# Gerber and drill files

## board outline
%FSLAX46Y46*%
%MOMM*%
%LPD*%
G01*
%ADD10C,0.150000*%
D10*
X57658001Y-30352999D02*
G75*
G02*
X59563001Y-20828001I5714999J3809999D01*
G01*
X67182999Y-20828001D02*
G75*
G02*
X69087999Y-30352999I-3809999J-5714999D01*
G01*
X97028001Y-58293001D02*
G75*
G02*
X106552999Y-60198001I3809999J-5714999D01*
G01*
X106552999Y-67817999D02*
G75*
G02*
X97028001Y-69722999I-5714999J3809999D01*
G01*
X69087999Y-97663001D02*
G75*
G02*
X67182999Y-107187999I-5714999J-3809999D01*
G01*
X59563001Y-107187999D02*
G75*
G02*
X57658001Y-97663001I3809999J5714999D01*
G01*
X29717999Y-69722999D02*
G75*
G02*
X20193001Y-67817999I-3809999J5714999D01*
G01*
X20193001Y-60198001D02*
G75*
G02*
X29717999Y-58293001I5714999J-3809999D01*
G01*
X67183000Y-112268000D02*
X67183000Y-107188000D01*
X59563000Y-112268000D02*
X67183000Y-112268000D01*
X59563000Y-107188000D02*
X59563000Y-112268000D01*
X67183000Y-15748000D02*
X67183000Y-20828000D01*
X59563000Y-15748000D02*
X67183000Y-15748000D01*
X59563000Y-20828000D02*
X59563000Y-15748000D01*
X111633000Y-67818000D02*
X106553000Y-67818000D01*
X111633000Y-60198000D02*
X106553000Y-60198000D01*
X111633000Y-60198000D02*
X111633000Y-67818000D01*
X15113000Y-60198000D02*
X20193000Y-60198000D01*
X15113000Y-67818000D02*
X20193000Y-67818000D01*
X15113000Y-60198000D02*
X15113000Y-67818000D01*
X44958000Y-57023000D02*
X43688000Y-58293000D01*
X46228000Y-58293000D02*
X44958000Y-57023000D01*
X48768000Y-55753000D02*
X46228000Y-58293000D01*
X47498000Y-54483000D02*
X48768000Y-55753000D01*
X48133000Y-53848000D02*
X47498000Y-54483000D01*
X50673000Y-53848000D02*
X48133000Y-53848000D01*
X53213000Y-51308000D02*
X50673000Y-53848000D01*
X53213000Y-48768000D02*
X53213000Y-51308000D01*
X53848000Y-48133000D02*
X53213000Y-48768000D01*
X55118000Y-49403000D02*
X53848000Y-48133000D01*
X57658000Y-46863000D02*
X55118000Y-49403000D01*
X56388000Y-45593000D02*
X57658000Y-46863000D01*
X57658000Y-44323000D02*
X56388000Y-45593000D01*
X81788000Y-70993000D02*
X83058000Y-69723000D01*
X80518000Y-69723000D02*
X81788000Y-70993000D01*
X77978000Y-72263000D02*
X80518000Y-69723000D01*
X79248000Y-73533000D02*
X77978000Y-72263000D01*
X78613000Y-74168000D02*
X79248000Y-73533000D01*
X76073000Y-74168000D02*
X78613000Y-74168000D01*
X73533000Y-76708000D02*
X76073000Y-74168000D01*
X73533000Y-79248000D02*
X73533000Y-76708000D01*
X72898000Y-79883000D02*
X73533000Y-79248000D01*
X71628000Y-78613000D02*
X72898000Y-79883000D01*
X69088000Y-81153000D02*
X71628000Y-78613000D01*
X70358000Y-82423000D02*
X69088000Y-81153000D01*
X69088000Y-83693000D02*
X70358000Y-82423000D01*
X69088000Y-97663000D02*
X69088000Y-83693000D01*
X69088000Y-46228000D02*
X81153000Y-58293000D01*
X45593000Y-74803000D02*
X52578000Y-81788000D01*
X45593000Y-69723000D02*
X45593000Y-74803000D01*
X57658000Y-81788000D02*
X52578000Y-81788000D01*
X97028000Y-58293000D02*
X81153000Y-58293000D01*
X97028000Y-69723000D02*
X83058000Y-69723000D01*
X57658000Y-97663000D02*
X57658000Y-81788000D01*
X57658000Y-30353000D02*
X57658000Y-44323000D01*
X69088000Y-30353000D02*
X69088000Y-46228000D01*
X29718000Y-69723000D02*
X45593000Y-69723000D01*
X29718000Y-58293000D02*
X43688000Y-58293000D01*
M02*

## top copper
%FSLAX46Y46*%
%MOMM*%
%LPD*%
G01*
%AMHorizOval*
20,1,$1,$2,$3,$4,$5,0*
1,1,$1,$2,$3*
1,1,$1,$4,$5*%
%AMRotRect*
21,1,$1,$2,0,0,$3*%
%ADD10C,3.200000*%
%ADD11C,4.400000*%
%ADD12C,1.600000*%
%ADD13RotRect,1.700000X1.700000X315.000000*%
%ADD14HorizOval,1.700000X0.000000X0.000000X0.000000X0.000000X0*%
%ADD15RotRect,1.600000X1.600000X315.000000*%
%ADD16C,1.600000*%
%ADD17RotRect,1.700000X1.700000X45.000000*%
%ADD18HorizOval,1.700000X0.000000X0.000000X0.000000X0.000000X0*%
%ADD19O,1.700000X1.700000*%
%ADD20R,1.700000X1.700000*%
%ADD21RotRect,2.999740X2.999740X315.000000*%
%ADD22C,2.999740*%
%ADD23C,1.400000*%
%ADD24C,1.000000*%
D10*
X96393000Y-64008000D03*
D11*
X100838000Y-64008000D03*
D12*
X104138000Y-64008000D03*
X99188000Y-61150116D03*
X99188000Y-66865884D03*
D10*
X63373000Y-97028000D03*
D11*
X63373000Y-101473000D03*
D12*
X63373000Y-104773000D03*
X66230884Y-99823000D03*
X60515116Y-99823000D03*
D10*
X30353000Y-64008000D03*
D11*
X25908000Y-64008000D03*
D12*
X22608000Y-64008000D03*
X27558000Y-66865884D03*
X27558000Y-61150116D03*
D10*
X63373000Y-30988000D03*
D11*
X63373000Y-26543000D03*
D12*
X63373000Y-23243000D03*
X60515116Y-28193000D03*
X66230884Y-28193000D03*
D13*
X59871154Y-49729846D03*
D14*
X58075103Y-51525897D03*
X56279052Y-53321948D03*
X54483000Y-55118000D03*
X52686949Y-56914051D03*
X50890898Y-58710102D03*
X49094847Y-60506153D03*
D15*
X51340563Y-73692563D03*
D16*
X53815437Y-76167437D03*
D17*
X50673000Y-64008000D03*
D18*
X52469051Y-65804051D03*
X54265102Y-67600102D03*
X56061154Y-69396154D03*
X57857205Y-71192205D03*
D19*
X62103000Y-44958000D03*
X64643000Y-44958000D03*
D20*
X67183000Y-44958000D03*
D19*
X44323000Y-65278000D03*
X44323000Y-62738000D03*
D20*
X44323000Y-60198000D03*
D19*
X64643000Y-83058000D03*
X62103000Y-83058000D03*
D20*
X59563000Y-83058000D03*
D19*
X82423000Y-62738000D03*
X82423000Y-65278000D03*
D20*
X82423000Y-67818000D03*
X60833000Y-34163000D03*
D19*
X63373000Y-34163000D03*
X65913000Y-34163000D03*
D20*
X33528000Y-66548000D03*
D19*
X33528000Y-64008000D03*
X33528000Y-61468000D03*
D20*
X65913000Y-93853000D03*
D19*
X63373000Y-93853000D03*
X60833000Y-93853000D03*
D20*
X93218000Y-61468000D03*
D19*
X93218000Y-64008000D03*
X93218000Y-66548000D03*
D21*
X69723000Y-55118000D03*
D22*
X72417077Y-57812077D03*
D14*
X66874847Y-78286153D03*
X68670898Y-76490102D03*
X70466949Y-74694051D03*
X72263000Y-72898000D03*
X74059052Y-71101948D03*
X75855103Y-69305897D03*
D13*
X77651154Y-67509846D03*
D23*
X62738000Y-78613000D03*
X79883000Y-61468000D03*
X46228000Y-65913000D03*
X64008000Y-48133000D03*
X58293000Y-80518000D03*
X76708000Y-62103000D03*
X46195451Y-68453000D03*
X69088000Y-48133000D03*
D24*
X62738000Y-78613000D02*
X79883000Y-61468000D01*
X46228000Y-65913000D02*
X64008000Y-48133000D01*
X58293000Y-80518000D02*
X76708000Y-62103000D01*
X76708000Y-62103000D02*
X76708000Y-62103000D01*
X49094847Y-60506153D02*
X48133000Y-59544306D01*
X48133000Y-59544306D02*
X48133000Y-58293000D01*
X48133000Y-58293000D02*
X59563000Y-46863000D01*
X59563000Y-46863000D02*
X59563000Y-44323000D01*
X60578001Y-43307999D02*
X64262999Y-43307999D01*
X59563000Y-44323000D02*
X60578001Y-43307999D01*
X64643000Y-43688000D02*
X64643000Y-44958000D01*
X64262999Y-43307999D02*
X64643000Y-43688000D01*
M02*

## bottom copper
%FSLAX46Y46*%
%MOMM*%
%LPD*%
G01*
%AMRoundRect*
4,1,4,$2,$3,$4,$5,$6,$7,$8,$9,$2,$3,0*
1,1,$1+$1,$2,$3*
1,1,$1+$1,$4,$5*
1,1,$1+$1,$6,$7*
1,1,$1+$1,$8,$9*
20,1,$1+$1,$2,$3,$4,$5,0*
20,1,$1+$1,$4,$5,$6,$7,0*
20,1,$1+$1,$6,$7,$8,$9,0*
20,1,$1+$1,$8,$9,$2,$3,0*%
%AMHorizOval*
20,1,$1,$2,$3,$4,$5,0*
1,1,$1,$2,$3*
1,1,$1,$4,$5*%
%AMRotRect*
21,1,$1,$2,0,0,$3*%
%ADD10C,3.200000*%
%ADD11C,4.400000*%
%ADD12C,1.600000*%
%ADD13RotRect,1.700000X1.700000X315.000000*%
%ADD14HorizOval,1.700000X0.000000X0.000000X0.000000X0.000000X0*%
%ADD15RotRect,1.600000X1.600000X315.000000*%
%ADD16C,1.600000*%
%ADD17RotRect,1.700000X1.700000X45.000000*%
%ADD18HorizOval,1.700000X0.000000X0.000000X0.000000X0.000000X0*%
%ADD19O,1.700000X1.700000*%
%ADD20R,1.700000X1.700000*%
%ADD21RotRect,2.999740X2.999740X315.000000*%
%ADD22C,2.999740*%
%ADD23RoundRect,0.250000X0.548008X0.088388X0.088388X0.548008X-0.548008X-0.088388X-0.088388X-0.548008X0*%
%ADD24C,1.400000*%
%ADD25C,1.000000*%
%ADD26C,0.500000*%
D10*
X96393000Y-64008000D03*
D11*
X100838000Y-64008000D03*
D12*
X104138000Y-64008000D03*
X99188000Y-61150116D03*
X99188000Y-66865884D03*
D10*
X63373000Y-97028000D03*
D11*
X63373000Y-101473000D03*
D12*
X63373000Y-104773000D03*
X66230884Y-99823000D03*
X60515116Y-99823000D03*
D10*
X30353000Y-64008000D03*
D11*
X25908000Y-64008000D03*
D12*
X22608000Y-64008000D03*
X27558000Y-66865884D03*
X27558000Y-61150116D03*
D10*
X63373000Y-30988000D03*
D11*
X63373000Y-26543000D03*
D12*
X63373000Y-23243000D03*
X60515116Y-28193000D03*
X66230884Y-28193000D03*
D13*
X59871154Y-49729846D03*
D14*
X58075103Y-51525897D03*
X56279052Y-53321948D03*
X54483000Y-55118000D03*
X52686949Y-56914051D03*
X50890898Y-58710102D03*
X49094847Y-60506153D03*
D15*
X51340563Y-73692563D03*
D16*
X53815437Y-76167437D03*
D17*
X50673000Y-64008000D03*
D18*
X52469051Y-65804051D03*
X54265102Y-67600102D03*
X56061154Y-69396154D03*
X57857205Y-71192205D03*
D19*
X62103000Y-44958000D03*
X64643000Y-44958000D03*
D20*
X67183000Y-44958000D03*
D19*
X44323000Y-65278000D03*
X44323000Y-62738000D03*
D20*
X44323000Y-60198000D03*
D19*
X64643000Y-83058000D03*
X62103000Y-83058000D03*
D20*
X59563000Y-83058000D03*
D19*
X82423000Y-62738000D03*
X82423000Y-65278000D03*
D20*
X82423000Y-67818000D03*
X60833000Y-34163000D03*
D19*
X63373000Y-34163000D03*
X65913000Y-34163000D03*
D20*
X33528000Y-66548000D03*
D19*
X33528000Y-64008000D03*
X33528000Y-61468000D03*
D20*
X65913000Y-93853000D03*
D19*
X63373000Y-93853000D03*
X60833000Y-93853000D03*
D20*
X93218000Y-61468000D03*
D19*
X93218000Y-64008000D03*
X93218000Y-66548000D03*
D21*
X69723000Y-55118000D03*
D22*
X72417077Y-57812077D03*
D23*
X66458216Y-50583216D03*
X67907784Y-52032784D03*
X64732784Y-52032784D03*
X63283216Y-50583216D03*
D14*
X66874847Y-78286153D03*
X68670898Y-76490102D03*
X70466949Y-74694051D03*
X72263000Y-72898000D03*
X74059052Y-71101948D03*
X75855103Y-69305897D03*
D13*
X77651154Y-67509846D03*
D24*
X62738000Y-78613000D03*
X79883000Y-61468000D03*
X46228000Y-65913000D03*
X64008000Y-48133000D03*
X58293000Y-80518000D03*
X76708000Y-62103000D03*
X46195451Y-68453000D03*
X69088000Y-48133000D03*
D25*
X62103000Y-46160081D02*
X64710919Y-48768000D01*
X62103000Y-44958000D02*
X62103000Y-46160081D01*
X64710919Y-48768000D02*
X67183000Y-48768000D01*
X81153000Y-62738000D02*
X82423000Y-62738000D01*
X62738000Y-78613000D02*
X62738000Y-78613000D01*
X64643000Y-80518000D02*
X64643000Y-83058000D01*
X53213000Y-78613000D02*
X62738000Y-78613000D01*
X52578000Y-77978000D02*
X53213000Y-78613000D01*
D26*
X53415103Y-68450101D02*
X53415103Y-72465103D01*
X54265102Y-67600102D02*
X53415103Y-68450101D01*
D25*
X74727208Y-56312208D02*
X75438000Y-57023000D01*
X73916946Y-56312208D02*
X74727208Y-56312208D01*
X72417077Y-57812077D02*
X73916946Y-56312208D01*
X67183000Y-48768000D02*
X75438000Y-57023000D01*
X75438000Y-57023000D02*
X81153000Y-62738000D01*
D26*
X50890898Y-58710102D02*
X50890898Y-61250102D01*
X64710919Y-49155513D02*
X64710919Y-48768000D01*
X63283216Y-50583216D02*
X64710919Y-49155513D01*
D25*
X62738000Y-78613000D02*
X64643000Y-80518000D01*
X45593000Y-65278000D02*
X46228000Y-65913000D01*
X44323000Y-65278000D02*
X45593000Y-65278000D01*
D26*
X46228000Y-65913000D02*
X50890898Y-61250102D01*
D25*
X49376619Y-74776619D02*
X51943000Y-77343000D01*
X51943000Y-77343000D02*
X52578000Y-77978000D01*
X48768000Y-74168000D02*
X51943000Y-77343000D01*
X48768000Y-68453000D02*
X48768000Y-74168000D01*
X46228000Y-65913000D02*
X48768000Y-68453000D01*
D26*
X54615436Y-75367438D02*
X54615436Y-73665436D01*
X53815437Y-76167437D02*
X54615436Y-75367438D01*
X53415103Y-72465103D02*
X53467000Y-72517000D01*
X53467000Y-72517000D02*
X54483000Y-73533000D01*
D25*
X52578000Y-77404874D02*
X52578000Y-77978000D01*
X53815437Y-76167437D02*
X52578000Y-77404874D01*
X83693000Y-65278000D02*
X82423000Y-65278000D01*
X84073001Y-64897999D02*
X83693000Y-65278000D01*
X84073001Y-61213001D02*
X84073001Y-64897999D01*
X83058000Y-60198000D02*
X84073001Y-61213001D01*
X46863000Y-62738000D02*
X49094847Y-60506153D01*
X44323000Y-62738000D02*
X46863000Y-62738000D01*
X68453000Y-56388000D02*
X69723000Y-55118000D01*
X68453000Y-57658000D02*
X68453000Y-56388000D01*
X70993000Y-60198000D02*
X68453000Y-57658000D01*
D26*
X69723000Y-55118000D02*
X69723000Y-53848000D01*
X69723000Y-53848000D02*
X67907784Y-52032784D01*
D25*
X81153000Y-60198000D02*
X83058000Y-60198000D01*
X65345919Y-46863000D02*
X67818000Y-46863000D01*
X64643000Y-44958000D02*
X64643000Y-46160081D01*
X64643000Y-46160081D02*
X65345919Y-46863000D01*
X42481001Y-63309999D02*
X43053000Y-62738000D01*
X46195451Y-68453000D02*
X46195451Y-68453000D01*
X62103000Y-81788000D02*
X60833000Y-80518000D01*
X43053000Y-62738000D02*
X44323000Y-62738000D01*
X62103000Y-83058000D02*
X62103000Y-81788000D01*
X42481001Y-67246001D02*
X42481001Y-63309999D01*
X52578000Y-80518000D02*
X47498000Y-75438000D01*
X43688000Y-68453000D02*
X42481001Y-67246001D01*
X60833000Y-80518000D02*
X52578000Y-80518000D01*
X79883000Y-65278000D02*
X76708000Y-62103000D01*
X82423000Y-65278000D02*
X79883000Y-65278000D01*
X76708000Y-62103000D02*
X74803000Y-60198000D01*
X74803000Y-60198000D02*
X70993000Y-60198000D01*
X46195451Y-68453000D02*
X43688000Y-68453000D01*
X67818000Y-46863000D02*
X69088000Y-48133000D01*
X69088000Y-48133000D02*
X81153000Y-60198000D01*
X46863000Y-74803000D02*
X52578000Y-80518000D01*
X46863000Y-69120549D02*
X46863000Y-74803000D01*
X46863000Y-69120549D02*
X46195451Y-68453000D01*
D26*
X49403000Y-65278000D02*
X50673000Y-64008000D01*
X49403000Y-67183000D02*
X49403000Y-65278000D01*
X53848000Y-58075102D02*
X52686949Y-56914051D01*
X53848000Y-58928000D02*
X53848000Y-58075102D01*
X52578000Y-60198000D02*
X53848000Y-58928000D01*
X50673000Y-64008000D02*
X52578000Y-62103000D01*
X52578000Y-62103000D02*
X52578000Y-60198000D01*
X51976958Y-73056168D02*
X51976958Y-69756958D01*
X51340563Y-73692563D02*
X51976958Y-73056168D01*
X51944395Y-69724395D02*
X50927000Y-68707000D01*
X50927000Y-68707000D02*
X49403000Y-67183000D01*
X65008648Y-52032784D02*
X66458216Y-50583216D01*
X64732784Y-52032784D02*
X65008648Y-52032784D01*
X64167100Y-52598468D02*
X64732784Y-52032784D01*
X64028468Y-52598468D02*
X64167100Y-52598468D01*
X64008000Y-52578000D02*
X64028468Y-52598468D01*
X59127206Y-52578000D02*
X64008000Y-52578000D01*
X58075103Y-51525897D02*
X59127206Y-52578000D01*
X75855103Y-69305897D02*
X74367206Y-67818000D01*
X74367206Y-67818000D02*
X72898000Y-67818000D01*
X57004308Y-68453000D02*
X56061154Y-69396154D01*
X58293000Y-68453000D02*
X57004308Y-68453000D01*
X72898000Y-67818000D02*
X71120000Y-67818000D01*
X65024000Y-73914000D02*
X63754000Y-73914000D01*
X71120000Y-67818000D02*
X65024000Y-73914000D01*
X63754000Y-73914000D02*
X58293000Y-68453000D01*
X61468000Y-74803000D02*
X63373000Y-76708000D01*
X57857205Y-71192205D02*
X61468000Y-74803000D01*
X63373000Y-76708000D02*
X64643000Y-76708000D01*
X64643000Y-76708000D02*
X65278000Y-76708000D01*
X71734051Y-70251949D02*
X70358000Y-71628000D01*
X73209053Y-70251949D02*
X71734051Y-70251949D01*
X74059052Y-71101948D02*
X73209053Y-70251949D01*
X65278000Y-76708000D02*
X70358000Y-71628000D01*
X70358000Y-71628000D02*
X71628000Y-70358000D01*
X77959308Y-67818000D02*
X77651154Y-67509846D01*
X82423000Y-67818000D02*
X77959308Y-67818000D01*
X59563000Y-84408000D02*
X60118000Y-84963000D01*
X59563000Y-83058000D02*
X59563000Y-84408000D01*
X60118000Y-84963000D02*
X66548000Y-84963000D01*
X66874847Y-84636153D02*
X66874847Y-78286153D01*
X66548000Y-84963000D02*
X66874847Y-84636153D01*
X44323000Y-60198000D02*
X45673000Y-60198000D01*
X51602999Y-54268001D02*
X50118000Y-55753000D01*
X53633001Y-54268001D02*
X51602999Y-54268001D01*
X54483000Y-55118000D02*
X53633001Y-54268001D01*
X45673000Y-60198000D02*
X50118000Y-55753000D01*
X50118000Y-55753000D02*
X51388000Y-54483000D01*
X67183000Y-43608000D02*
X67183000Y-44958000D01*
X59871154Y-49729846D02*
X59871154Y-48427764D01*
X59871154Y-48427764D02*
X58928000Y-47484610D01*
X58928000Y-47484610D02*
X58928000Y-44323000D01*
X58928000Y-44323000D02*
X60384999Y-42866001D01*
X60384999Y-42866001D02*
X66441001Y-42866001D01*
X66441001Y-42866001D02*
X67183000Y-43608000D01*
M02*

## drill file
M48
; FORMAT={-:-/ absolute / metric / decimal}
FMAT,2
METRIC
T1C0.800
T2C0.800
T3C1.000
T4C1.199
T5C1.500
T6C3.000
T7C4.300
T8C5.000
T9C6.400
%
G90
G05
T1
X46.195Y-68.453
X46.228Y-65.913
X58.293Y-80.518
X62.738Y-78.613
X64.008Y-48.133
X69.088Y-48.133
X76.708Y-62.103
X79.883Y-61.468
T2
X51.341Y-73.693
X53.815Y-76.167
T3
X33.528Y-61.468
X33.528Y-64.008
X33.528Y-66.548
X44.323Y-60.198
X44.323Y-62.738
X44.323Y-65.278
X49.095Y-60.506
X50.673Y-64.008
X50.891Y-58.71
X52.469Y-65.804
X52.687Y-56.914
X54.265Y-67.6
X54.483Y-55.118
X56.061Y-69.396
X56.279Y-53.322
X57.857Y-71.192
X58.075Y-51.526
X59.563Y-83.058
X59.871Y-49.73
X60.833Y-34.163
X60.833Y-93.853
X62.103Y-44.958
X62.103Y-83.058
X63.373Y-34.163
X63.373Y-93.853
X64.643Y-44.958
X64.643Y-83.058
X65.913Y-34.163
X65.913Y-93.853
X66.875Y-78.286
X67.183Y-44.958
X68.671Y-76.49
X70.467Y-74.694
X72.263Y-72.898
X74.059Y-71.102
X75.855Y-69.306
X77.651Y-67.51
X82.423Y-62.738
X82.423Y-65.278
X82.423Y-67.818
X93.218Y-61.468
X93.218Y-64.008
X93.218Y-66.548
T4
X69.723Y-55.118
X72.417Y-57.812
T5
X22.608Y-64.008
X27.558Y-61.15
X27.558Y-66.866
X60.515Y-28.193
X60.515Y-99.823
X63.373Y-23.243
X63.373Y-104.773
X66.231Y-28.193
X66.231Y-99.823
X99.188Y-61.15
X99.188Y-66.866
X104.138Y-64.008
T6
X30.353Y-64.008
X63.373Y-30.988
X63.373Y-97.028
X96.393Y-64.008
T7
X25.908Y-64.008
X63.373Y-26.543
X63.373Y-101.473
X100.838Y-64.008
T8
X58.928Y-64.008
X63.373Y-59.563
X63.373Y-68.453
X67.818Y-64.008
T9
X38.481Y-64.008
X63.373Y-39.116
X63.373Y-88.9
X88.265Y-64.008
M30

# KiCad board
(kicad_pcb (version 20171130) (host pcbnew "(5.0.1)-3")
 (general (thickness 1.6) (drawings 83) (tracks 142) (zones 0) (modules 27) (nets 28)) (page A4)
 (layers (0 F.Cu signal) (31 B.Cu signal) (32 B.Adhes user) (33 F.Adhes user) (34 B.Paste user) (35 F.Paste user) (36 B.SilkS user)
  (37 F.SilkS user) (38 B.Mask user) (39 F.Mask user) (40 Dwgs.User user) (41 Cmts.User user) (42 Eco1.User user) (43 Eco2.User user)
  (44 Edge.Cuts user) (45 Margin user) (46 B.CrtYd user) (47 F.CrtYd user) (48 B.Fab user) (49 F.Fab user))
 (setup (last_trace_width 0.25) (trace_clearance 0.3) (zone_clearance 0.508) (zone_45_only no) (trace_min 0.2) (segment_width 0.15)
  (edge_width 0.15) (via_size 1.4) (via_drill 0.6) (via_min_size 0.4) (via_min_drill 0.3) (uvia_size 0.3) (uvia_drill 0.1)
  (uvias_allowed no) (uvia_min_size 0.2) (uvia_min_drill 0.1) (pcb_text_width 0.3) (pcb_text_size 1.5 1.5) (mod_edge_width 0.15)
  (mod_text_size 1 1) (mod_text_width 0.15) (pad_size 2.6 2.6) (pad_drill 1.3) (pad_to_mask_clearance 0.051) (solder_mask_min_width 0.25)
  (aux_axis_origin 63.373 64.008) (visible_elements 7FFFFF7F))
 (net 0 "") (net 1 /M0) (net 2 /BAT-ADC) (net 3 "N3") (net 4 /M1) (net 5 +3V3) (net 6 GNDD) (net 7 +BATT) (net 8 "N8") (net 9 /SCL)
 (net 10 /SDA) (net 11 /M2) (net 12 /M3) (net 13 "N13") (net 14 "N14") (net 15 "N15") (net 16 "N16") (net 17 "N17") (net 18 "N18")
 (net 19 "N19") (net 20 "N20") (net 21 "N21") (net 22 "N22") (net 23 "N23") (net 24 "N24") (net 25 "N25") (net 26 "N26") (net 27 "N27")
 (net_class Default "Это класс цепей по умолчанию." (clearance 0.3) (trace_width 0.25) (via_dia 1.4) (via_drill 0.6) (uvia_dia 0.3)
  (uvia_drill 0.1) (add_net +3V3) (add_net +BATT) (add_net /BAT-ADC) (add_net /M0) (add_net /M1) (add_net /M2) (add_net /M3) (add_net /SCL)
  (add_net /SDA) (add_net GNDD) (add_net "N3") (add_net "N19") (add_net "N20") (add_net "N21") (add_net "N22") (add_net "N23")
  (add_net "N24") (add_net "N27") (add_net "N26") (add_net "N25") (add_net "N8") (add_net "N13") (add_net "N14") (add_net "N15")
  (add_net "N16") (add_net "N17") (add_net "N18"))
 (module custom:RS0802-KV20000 (layer F.Cu) (at 100.838 64.008)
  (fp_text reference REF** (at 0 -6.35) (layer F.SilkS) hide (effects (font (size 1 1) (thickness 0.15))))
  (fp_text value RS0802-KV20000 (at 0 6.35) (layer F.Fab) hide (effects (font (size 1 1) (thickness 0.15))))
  (pad "" np_thru_hole circle (at -4.445 0) (size 3.2 3.2) (drill 3) (layers *.Cu *.Mask))
  (pad "" np_thru_hole circle (at 0 0) (size 4.4 4.4) (drill 4.3) (layers *.Cu *.Mask))
  (pad "" np_thru_hole circle (at 3.3 0) (size 1.6 1.6) (drill 1.5) (layers *.Cu *.Mask))
  (pad "" np_thru_hole circle (at -1.65 -2.857884 120) (size 1.6 1.6) (drill 1.5) (layers *.Cu *.Mask))
  (pad "" np_thru_hole circle (at -1.65 2.857884 240) (size 1.6 1.6) (drill 1.5) (layers *.Cu *.Mask)))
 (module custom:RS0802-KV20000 (layer F.Cu) (at 63.373 101.473 270)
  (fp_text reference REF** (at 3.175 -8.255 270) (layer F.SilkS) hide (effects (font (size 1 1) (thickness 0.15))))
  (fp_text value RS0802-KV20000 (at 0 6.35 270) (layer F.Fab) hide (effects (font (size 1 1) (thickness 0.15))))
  (pad "" np_thru_hole circle (at -4.445 0 270) (size 3.2 3.2) (drill 3) (layers *.Cu *.Mask))
  (pad "" np_thru_hole circle (at 0 0 270) (size 4.4 4.4) (drill 4.3) (layers *.Cu *.Mask))
  (pad "" np_thru_hole circle (at 3.3 0 270) (size 1.6 1.6) (drill 1.5) (layers *.Cu *.Mask))
  (pad "" np_thru_hole circle (at -1.65 -2.857884 30) (size 1.6 1.6) (drill 1.5) (layers *.Cu *.Mask))
  (pad "" np_thru_hole circle (at -1.65 2.857884 150) (size 1.6 1.6) (drill 1.5) (layers *.Cu *.Mask)))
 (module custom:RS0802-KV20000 (layer F.Cu) (at 25.908 64.008 180)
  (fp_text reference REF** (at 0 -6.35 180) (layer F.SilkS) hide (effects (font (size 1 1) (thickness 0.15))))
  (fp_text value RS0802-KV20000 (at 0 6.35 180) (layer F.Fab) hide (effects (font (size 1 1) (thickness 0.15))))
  (pad "" np_thru_hole circle (at -4.445 0 180) (size 3.2 3.2) (drill 3) (layers *.Cu *.Mask))
  (pad "" np_thru_hole circle (at 0 0 180) (size 4.4 4.4) (drill 4.3) (layers *.Cu *.Mask))
  (pad "" np_thru_hole circle (at 3.3 0 180) (size 1.6 1.6) (drill 1.5) (layers *.Cu *.Mask))
  (pad "" np_thru_hole circle (at -1.65 -2.857884 300) (size 1.6 1.6) (drill 1.5) (layers *.Cu *.Mask))
  (pad "" np_thru_hole circle (at -1.65 2.857884 60) (size 1.6 1.6) (drill 1.5) (layers *.Cu *.Mask)))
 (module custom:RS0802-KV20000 (layer F.Cu) (at 63.373 26.543 90)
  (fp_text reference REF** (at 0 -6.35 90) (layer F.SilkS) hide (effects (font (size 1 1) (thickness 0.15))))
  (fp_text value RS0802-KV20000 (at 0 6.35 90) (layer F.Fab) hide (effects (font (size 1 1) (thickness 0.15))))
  (pad "" np_thru_hole circle (at -4.445 0 90) (size 3.2 3.2) (drill 3) (layers *.Cu *.Mask))
  (pad "" np_thru_hole circle (at 0 0 90) (size 4.4 4.4) (drill 4.3) (layers *.Cu *.Mask))
  (pad "" np_thru_hole circle (at 3.3 0 90) (size 1.6 1.6) (drill 1.5) (layers *.Cu *.Mask))
  (pad "" np_thru_hole circle (at -1.65 -2.857884 210) (size 1.6 1.6) (drill 1.5) (layers *.Cu *.Mask))
  (pad "" np_thru_hole circle (at -1.65 2.857884 330) (size 1.6 1.6) (drill 1.5) (layers *.Cu *.Mask)))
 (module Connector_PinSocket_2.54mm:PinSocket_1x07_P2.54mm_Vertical (layer F.Cu) (at 59.871154 49.729846 315)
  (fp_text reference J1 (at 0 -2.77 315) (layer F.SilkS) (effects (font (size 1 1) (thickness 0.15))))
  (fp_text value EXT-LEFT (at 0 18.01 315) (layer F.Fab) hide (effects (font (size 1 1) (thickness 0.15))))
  (pad 1 thru_hole rect (at 0 0 315) (size 1.7 1.7) (drill 1) (layers *.Cu *.Mask) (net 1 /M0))
  (pad 2 thru_hole oval (at 0 2.54 315) (size 1.7 1.7) (drill 1) (layers *.Cu *.Mask) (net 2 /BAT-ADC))
  (pad 3 thru_hole oval (at 0 5.079999 315) (size 1.7 1.7) (drill 1) (layers *.Cu *.Mask) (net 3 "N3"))
  (pad 4 thru_hole oval (at 0 7.62 315) (size 1.7 1.7) (drill 1) (layers *.Cu *.Mask) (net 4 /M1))
  (pad 5 thru_hole oval (at 0 10.16 315) (size 1.7 1.7) (drill 1) (layers *.Cu *.Mask) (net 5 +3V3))
  (pad 6 thru_hole oval (at 0 12.7 315) (size 1.7 1.7) (drill 1) (layers *.Cu *.Mask) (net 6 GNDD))
  (pad 7 thru_hole oval (at 0 15.24 315) (size 1.7 1.7) (drill 1) (layers *.Cu *.Mask) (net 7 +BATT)))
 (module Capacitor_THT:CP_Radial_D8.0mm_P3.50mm (layer F.Cu) (at 52.578 74.93 315)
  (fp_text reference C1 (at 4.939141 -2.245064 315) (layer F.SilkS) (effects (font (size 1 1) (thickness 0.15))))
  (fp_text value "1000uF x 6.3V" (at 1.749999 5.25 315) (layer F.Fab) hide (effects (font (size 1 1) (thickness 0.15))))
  (pad 1 thru_hole rect (at -1.75 0 315) (size 1.6 1.6) (drill 0.8) (layers *.Cu *.Mask) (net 5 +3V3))
  (pad 2 thru_hole circle (at 1.75 0 315) (size 1.6 1.6) (drill 0.8) (layers *.Cu *.Mask) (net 6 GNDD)))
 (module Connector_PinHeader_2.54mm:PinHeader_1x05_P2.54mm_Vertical (layer F.Cu) (at 50.673 64.008 45)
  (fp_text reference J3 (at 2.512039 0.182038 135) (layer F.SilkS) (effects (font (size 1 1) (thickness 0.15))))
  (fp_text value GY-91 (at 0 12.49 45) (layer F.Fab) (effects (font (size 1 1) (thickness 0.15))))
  (pad 1 thru_hole rect (at 0 0 45) (size 1.7 1.7) (drill 1) (layers *.Cu *.Mask) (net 5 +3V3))
  (pad 2 thru_hole oval (at 0 2.54 45) (size 1.7 1.7) (drill 1) (layers *.Cu *.Mask) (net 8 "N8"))
  (pad 3 thru_hole oval (at 0 5.079999 45) (size 1.7 1.7) (drill 1) (layers *.Cu *.Mask) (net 6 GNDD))
  (pad 4 thru_hole oval (at 0 7.62 45) (size 1.7 1.7) (drill 1) (layers *.Cu *.Mask) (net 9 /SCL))
  (pad 5 thru_hole oval (at 0 10.16 45) (size 1.7 1.7) (drill 1) (layers *.Cu *.Mask) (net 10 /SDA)))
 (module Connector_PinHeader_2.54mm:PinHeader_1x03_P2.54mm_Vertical (layer F.Cu) (at 67.183 44.958 270)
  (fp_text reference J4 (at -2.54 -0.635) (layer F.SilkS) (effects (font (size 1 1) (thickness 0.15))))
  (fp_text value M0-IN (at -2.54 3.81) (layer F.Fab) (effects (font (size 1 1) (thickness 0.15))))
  (pad 3 thru_hole oval (at 0 5.08 270) (size 1.7 1.7) (drill 1) (layers *.Cu *.Mask) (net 6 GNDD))
  (pad 2 thru_hole oval (at 0 2.54 270) (size 1.7 1.7) (drill 1) (layers *.Cu *.Mask) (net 7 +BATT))
  (pad 1 thru_hole rect (at 0 0 270) (size 1.7 1.7) (drill 1) (layers *.Cu *.Mask) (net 1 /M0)))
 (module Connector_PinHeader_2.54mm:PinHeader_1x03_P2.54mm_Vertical (layer F.Cu) (at 44.323 60.198)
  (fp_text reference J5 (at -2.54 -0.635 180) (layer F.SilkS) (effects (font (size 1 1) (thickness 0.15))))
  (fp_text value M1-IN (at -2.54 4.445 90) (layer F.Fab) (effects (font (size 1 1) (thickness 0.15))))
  (pad 3 thru_hole oval (at 0 5.08) (size 1.7 1.7) (drill 1) (layers *.Cu *.Mask) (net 6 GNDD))
  (pad 2 thru_hole oval (at 0 2.54) (size 1.7 1.7) (drill 1) (layers *.Cu *.Mask) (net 7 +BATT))
  (pad 1 thru_hole rect (at 0 0) (size 1.7 1.7) (drill 1) (layers *.Cu *.Mask) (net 4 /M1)))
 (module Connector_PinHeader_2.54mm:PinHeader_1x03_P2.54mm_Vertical (layer F.Cu) (at 59.563 83.058 90)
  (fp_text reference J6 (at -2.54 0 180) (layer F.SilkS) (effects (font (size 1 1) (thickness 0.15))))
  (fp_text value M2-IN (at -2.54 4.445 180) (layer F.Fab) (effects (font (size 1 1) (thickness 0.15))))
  (pad 3 thru_hole oval (at 0 5.08 90) (size 1.7 1.7) (drill 1) (layers *.Cu *.Mask) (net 6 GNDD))
  (pad 2 thru_hole oval (at 0 2.54 90) (size 1.7 1.7) (drill 1) (layers *.Cu *.Mask) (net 7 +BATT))
  (pad 1 thru_hole rect (at 0 0 90) (size 1.7 1.7) (drill 1) (layers *.Cu *.Mask) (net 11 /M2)))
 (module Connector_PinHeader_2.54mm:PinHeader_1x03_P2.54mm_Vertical (layer F.Cu) (at 82.423 67.818 180)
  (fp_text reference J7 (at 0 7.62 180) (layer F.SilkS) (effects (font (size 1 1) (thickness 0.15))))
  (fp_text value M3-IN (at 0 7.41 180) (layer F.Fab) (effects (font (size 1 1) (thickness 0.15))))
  (pad 3 thru_hole oval (at 0 5.08 180) (size 1.7 1.7) (drill 1) (layers *.Cu *.Mask) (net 6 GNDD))
  (pad 2 thru_hole oval (at 0 2.54 180) (size 1.7 1.7) (drill 1) (layers *.Cu *.Mask) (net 7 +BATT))
  (pad 1 thru_hole rect (at 0 0 180) (size 1.7 1.7) (drill 1) (layers *.Cu *.Mask) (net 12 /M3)))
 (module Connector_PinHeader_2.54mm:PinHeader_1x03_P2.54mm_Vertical (layer F.Cu) (at 60.833 34.163 90)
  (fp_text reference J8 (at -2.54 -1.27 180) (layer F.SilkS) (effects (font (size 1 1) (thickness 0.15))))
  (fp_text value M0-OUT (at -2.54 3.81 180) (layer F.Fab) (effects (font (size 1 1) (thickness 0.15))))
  (pad 1 thru_hole rect (at 0 0 90) (size 1.7 1.7) (drill 1) (layers *.Cu *.Mask) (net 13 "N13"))
  (pad 2 thru_hole oval (at 0 2.54 90) (size 1.7 1.7) (drill 1) (layers *.Cu *.Mask) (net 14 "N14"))
  (pad 3 thru_hole oval (at 0 5.08 90) (size 1.7 1.7) (drill 1) (layers *.Cu *.Mask) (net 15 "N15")))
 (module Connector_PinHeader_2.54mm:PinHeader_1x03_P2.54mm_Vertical (layer F.Cu) (at 33.528 66.548 180)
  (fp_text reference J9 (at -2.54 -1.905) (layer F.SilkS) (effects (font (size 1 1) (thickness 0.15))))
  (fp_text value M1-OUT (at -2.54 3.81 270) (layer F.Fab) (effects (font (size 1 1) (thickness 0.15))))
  (pad 1 thru_hole rect (at 0 0 180) (size 1.7 1.7) (drill 1) (layers *.Cu *.Mask) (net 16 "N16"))
  (pad 2 thru_hole oval (at 0 2.54 180) (size 1.7 1.7) (drill 1) (layers *.Cu *.Mask) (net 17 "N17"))
  (pad 3 thru_hole oval (at 0 5.08 180) (size 1.7 1.7) (drill 1) (layers *.Cu *.Mask) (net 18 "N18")))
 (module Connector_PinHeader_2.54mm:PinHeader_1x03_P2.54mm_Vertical (layer F.Cu) (at 65.913 93.853 270)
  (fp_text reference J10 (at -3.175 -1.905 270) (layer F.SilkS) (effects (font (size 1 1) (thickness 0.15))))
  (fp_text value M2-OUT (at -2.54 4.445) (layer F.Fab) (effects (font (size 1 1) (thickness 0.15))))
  (pad 1 thru_hole rect (at 0 0 270) (size 1.7 1.7) (drill 1) (layers *.Cu *.Mask) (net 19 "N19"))
  (pad 2 thru_hole oval (at 0 2.54 270) (size 1.7 1.7) (drill 1) (layers *.Cu *.Mask) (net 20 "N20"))
  (pad 3 thru_hole oval (at 0 5.08 270) (size 1.7 1.7) (drill 1) (layers *.Cu *.Mask) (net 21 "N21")))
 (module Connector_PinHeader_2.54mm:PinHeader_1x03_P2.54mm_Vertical (layer F.Cu) (at 93.218 61.468)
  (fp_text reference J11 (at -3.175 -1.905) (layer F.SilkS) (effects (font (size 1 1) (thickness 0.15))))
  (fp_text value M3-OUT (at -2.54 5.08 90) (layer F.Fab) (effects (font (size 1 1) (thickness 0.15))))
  (pad 1 thru_hole rect (at 0 0) (size 1.7 1.7) (drill 1) (layers *.Cu *.Mask) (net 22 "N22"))
  (pad 2 thru_hole oval (at 0 2.54) (size 1.7 1.7) (drill 1) (layers *.Cu *.Mask) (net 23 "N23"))
  (pad 3 thru_hole oval (at 0 5.08) (size 1.7 1.7) (drill 1) (layers *.Cu *.Mask) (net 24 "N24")))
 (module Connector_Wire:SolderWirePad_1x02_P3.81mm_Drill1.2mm (layer F.Cu) (at 69.723 55.118 315)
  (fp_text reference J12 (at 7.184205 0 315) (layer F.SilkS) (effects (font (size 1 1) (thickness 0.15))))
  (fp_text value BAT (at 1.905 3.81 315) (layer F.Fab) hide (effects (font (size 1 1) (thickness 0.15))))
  (pad 1 thru_hole rect (at 0 0 315) (size 2.99974 2.99974) (drill 1.19888) (layers *.Cu *.Mask) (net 7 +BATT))
  (pad 2 thru_hole circle (at 3.81 0 315) (size 2.99974 2.99974) (drill 1.19888) (layers *.Cu *.Mask) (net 6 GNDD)))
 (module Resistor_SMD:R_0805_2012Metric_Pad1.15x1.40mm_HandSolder (layer B.Cu) (at 67.183 51.308 135)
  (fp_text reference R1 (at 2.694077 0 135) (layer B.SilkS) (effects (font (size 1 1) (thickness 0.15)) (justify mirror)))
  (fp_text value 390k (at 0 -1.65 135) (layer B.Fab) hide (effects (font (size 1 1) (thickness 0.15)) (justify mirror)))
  (pad 2 smd roundrect (at 1.024999 0 135) (size 1.15 1.4) (layers B.Cu B.Paste B.Mask) (roundrect_rratio 0.217391) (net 2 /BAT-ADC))
  (pad 1 smd roundrect (at -1.024999 0 135) (size 1.15 1.4) (layers B.Cu B.Paste B.Mask) (roundrect_rratio 0.217391) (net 7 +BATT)))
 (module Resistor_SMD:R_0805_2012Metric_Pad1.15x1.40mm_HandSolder (layer B.Cu) (at 64.008 51.308 135)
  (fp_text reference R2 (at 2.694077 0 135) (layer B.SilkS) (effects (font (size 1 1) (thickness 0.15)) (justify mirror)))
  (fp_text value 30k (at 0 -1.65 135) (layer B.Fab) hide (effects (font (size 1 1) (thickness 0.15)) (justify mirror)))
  (pad 1 smd roundrect (at -1.024999 0 135) (size 1.15 1.4) (layers B.Cu B.Paste B.Mask) (roundrect_rratio 0.217391) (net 2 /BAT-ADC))
  (pad 2 smd roundrect (at 1.024999 0 135) (size 1.15 1.4) (layers B.Cu B.Paste B.Mask) (roundrect_rratio 0.217391) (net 6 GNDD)))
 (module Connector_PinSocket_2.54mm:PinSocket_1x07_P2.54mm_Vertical (layer F.Cu) (at 77.651154 67.509846 315)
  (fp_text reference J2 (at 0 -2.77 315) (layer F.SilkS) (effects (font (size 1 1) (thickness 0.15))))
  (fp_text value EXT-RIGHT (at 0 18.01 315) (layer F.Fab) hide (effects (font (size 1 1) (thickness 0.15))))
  (pad 7 thru_hole oval (at 0 15.24 315) (size 1.7 1.7) (drill 1) (layers *.Cu *.Mask) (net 11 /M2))
  (pad 6 thru_hole oval (at 0 12.7 315) (size 1.7 1.7) (drill 1) (layers *.Cu *.Mask) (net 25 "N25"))
  (pad 5 thru_hole oval (at 0 10.16 315) (size 1.7 1.7) (drill 1) (layers *.Cu *.Mask) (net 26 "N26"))
  (pad 4 thru_hole oval (at 0 7.62 315) (size 1.7 1.7) (drill 1) (layers *.Cu *.Mask) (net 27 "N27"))
  (pad 3 thru_hole oval (at 0 5.079999 315) (size 1.7 1.7) (drill 1) (layers *.Cu *.Mask) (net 10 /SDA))
  (pad 2 thru_hole oval (at 0 2.54 315) (size 1.7 1.7) (drill 1) (layers *.Cu *.Mask) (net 9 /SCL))
  (pad 1 thru_hole rect (at 0 0 315) (size 1.7 1.7) (drill 1) (layers *.Cu *.Mask) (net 12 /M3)))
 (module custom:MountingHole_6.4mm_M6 (layer F.Cu) (at 38.481 64.008)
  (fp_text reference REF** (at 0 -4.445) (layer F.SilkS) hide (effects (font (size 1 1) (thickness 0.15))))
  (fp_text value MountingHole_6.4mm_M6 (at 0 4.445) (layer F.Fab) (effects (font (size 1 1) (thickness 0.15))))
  (pad 1 np_thru_hole circle (at 0 0) (size 6.4 6.4) (drill 6.4) (layers *.Cu *.Mask)))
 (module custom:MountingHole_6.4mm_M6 (layer F.Cu) (at 63.373 88.9)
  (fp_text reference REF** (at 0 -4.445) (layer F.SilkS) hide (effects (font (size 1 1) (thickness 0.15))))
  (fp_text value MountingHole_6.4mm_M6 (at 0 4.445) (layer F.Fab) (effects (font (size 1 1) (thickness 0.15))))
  (pad 1 np_thru_hole circle (at 0 0) (size 6.4 6.4) (drill 6.4) (layers *.Cu *.Mask)))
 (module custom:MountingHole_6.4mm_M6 (layer F.Cu) (at 88.265 64.008)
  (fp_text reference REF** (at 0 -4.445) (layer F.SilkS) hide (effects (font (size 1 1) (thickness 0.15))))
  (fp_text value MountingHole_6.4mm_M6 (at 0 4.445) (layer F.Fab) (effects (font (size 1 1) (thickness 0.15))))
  (pad 1 np_thru_hole circle (at 0 0) (size 6.4 6.4) (drill 6.4) (layers *.Cu *.Mask)))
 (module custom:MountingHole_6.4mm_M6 (layer F.Cu) (at 63.373 39.116)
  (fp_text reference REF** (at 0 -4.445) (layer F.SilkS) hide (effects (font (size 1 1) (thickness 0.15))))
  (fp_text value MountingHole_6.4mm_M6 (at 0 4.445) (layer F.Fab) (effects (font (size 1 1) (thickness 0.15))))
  (pad 1 np_thru_hole circle (at 0 0) (size 6.4 6.4) (drill 6.4) (layers *.Cu *.Mask)))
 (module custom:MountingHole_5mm (layer F.Cu) (at 63.373 68.453)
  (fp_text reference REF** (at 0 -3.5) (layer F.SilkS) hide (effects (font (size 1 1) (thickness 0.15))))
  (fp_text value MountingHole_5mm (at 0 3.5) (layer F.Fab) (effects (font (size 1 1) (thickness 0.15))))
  (pad "" np_thru_hole circle (at 0 0) (size 5 5) (drill 5) (layers *.Cu *.Mask)))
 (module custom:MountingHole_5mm (layer F.Cu) (at 58.928 64.008)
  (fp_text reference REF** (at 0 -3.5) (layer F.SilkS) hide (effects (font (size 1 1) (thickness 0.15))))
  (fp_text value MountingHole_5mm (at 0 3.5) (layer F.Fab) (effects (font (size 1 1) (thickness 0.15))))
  (pad "" np_thru_hole circle (at 0 0) (size 5 5) (drill 5) (layers *.Cu *.Mask)))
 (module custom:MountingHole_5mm (layer F.Cu) (at 63.373 59.563)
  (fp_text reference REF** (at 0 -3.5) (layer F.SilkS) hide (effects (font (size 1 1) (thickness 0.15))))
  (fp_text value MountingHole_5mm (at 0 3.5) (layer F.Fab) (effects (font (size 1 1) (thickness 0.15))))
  (pad "" np_thru_hole circle (at 0 0) (size 5 5) (drill 5) (layers *.Cu *.Mask)))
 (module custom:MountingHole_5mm (layer F.Cu) (at 67.818 64.008)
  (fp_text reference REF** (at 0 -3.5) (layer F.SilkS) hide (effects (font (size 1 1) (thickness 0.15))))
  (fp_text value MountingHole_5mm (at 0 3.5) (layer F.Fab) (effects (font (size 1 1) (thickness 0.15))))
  (pad "" np_thru_hole circle (at 0 0) (size 5 5) (drill 5) (layers *.Cu *.Mask)))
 (gr_arc (start 63.373 26.543) (end 59.563001 20.828001) (angle -90) (layer Edge.Cuts) (width 0.15))
 (gr_arc (start 63.373 26.543) (end 69.087999 30.352999) (angle -90) (layer Edge.Cuts) (width 0.15))
 (gr_arc (start 100.838 64.008) (end 106.552999 60.198001) (angle -90) (layer Edge.Cuts) (width 0.15))
 (gr_arc (start 100.838 64.008) (end 97.028001 69.722999) (angle -90) (layer Edge.Cuts) (width 0.15))
 (gr_arc (start 63.373 101.473) (end 67.182999 107.187999) (angle -90) (layer Edge.Cuts) (width 0.15))
 (gr_arc (start 63.373 101.473) (end 57.658001 97.663001) (angle -90) (layer Edge.Cuts) (width 0.15))
 (gr_arc (start 25.908 64.008) (end 20.193001 67.817999) (angle -90) (layer Edge.Cuts) (width 0.15))
 (gr_arc (start 25.908 64.008) (end 29.717999 58.293001) (angle -90) (layer Edge.Cuts) (width 0.15))
 (gr_line (start 67.183 112.268) (end 67.183 107.188) (layer Edge.Cuts) (width 0.15))
 (gr_line (start 59.563 112.268) (end 67.183 112.268) (layer Edge.Cuts) (width 0.15))
 (gr_line (start 59.563 107.188) (end 59.563 112.268) (layer Edge.Cuts) (width 0.15))
 (gr_line (start 67.183 15.748) (end 67.183 20.828) (layer Edge.Cuts) (width 0.15))
 (gr_line (start 59.563 15.748) (end 67.183 15.748) (layer Edge.Cuts) (width 0.15))
 (gr_line (start 59.563 20.828) (end 59.563 15.748) (layer Edge.Cuts) (width 0.15))
 (gr_line (start 111.633 67.818) (end 106.553 67.818) (layer Edge.Cuts) (width 0.15))
 (gr_line (start 111.633 60.198) (end 106.553 60.198) (layer Edge.Cuts) (width 0.15))
 (gr_line (start 111.633 60.198) (end 111.633 67.818) (layer Edge.Cuts) (width 0.15))
 (gr_line (start 15.113 60.198) (end 20.193 60.198) (layer Edge.Cuts) (width 0.15))
 (gr_line (start 15.113 67.818) (end 20.193 67.818) (layer Edge.Cuts) (width 0.15))
 (gr_line (start 15.113 60.198) (end 15.113 67.818) (layer Edge.Cuts) (width 0.15))
 (gr_line (start 44.958 57.023) (end 43.688 58.293) (layer Edge.Cuts) (width 0.15))
 (gr_line (start 46.228 58.293) (end 44.958 57.023) (layer Edge.Cuts) (width 0.15))
 (gr_line (start 48.768 55.753) (end 46.228 58.293) (layer Edge.Cuts) (width 0.15))
 (gr_line (start 47.498 54.483) (end 48.768 55.753) (layer Edge.Cuts) (width 0.15))
 (gr_line (start 48.133 53.848) (end 47.498 54.483) (layer Edge.Cuts) (width 0.15))
 (gr_line (start 50.673 53.848) (end 48.133 53.848) (layer Edge.Cuts) (width 0.15))
 (gr_line (start 53.213 51.308) (end 50.673 53.848) (layer Edge.Cuts) (width 0.15))
 (gr_line (start 53.213 48.768) (end 53.213 51.308) (layer Edge.Cuts) (width 0.15))
 (gr_line (start 53.848 48.133) (end 53.213 48.768) (layer Edge.Cuts) (width 0.15))
 (gr_line (start 55.118 49.403) (end 53.848 48.133) (layer Edge.Cuts) (width 0.15))
 (gr_line (start 57.658 46.863) (end 55.118 49.403) (layer Edge.Cuts) (width 0.15))
 (gr_line (start 56.388 45.593) (end 57.658 46.863) (layer Edge.Cuts) (width 0.15))
 (gr_line (start 57.658 44.323) (end 56.388 45.593) (layer Edge.Cuts) (width 0.15))
 (gr_line (start 81.788 70.993) (end 83.058 69.723) (layer Edge.Cuts) (width 0.15))
 (gr_line (start 80.518 69.723) (end 81.788 70.993) (layer Edge.Cuts) (width 0.15))
 (gr_line (start 77.978 72.263) (end 80.518 69.723) (layer Edge.Cuts) (width 0.15))
 (gr_line (start 79.248 73.533) (end 77.978 72.263) (layer Edge.Cuts) (width 0.15))
 (gr_line (start 78.613 74.168) (end 79.248 73.533) (layer Edge.Cuts) (width 0.15))
 (gr_line (start 76.073 74.168) (end 78.613 74.168) (layer Edge.Cuts) (width 0.15))
 (gr_line (start 73.533 76.708) (end 76.073 74.168) (layer Edge.Cuts) (width 0.15))
 (gr_line (start 73.533 79.248) (end 73.533 76.708) (layer Edge.Cuts) (width 0.15))
 (gr_line (start 72.898 79.883) (end 73.533 79.248) (layer Edge.Cuts) (width 0.15))
 (gr_line (start 71.628 78.613) (end 72.898 79.883) (layer Edge.Cuts) (width 0.15))
 (gr_line (start 69.088 81.153) (end 71.628 78.613) (layer Edge.Cuts) (width 0.15))
 (gr_line (start 70.358 82.423) (end 69.088 81.153) (layer Edge.Cuts) (width 0.15))
 (gr_line (start 69.088 83.693) (end 70.358 82.423) (layer Edge.Cuts) (width 0.15))
 (gr_line (start 69.088 97.663) (end 69.088 83.693) (layer Edge.Cuts) (width 0.15))
 (gr_line (start 69.088 46.228) (end 81.153 58.293) (layer Edge.Cuts) (width 0.15))
 (gr_line (start 45.593 74.803) (end 52.578 81.788) (layer Edge.Cuts) (width 0.15))
 (gr_line (start 45.593 69.723) (end 45.593 74.803) (layer Edge.Cuts) (width 0.15))
 (gr_line (start 57.658 81.788) (end 52.578 81.788) (layer Edge.Cuts) (width 0.15))
 (gr_line (start 97.028 58.293) (end 81.153 58.293) (layer Edge.Cuts) (width 0.15))
 (gr_line (start 97.028 69.723) (end 83.058 69.723) (layer Edge.Cuts) (width 0.15))
 (gr_line (start 57.658 97.663) (end 57.658 81.788) (layer Edge.Cuts) (width 0.15))
 (gr_line (start 57.658 30.353) (end 57.658 44.323) (layer Edge.Cuts) (width 0.15))
 (gr_line (start 69.088 30.353) (end 69.088 46.228) (layer Edge.Cuts) (width 0.15))
 (gr_line (start 29.718 69.723) (end 45.593 69.723) (layer Edge.Cuts) (width 0.15))
 (gr_line (start 29.718 58.293) (end 43.688 58.293) (layer Edge.Cuts) (width 0.15))
 (segment (start 62.103 46.160081) (end 64.710919 48.768) (width 1) (layer B.Cu) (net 6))
 (segment (start 62.103 44.958) (end 62.103 46.160081) (width 1) (layer B.Cu) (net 6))
 (segment (start 64.710919 48.768) (end 67.183 48.768) (width 1) (layer B.Cu) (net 6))
 (segment (start 81.153 62.738) (end 82.423 62.738) (width 1) (layer B.Cu) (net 6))
 (segment (start 62.738 78.613) (end 62.738 78.613) (width 1) (layer B.Cu) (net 6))
 (segment (start 64.643 80.518) (end 64.643 83.058) (width 1) (layer B.Cu) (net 6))
 (segment (start 53.213 78.613) (end 62.738 78.613) (width 1) (layer B.Cu) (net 6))
 (segment (start 52.578 77.978) (end 53.213 78.613) (width 1) (layer B.Cu) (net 6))
 (segment (start 53.415103 68.450101) (end 53.415103 72.465103) (width 0.5) (layer B.Cu) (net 6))
 (segment (start 54.265102 67.600102) (end 53.415103 68.450101) (width 0.5) (layer B.Cu) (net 6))
 (segment (start 74.727208 56.312208) (end 75.438 57.023) (width 1) (layer B.Cu) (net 6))
 (segment (start 73.916946 56.312208) (end 74.727208 56.312208) (width 1) (layer B.Cu) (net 6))
 (segment (start 72.417077 57.812077) (end 73.916946 56.312208) (width 1) (layer B.Cu) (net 6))
 (segment (start 67.183 48.768) (end 75.438 57.023) (width 1) (layer B.Cu) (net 6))
 (segment (start 75.438 57.023) (end 81.153 62.738) (width 1) (layer B.Cu) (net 6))
 (segment (start 50.890898 58.710102) (end 50.890898 61.250102) (width 0.5) (layer B.Cu) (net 6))
 (segment (start 64.710919 49.155513) (end 64.710919 48.768) (width 0.5) (layer B.Cu) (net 6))
 (segment (start 63.283216 50.583216) (end 64.710919 49.155513) (width 0.5) (layer B.Cu) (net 6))
 (segment (start 62.738 78.613) (end 64.643 80.518) (width 1) (layer B.Cu) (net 6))
 (via (at 62.738 78.613) (size 1.4) (drill 0.8) (layers F.Cu B.Cu) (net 6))
 (segment (start 62.738 78.613) (end 79.883 61.468) (width 1) (layer F.Cu) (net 6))
 (via (at 79.883 61.468) (size 1.4) (drill 0.8) (layers F.Cu B.Cu) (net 6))
 (via (at 46.228 65.913) (size 1.4) (drill 0.8) (layers F.Cu B.Cu) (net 6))
 (segment (start 45.593 65.278) (end 46.228 65.913) (width 1) (layer B.Cu) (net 6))
 (segment (start 44.323 65.278) (end 45.593 65.278) (width 1) (layer B.Cu) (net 6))
 (segment (start 46.228 65.913) (end 50.890898 61.250102) (width 0.5) (layer B.Cu) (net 6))
 (via (at 64.008 48.133) (size 1.4) (drill 0.8) (layers F.Cu B.Cu) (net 6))
 (segment (start 46.228 65.913) (end 64.008 48.133) (width 1) (layer F.Cu) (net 6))
 (segment (start 49.376619 74.776619) (end 51.943 77.343) (width 1) (layer B.Cu) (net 6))
 (segment (start 51.943 77.343) (end 52.578 77.978) (width 1) (layer B.Cu) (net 6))
 (segment (start 48.768 74.168) (end 51.943 77.343) (width 1) (layer B.Cu) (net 6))
 (segment (start 48.768 68.453) (end 48.768 74.168) (width 1) (layer B.Cu) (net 6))
 (segment (start 46.228 65.913) (end 48.768 68.453) (width 1) (layer B.Cu) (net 6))
 (segment (start 54.615436 75.367438) (end 54.615436 73.665436) (width 0.5) (layer B.Cu) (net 6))
 (segment (start 53.815437 76.167437) (end 54.615436 75.367438) (width 0.5) (layer B.Cu) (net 6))
 (segment (start 53.415103 72.465103) (end 53.467 72.517) (width 0.5) (layer B.Cu) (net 6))
 (segment (start 53.467 72.517) (end 54.483 73.533) (width 0.5) (layer B.Cu) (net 6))
 (segment (start 52.578 77.404874) (end 52.578 77.978) (width 1) (layer B.Cu) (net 6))
 (segment (start 53.815437 76.167437) (end 52.578 77.404874) (width 1) (layer B.Cu) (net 6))
 (segment (start 83.693 65.278) (end 82.423 65.278) (width 1) (layer B.Cu) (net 7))
 (segment (start 84.073001 64.897999) (end 83.693 65.278) (width 1) (layer B.Cu) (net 7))
 (segment (start 84.073001 61.213001) (end 84.073001 64.897999) (width 1) (layer B.Cu) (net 7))
 (segment (start 83.058 60.198) (end 84.073001 61.213001) (width 1) (layer B.Cu) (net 7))
 (segment (start 46.863 62.738) (end 49.094847 60.506153) (width 1) (layer B.Cu) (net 7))
 (segment (start 44.323 62.738) (end 46.863 62.738) (width 1) (layer B.Cu) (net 7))
 (segment (start 68.453 56.388) (end 69.723 55.118) (width 1) (layer B.Cu) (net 7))
 (segment (start 68.453 57.658) (end 68.453 56.388) (width 1) (layer B.Cu) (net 7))
 (segment (start 70.993 60.198) (end 68.453 57.658) (width 1) (layer B.Cu) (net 7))
 (segment (start 69.723 55.118) (end 69.723 53.848) (width 0.5) (layer B.Cu) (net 7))
 (segment (start 69.723 53.848) (end 67.907784 52.032784) (width 0.5) (layer B.Cu) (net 7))
 (via (at 58.293 80.518) (size 1.4) (drill 0.8) (layers F.Cu B.Cu) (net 7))
 (segment (start 81.153 60.198) (end 83.058 60.198) (width 1) (layer B.Cu) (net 7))
 (segment (start 65.345919 46.863) (end 67.818 46.863) (width 1) (layer B.Cu) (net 7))
 (segment (start 64.643 44.958) (end 64.643 46.160081) (width 1) (layer B.Cu) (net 7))
 (segment (start 64.643 46.160081) (end 65.345919 46.863) (width 1) (layer B.Cu) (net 7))
 (segment (start 42.481001 63.309999) (end 43.053 62.738) (width 1) (layer B.Cu) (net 7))
 (segment (start 46.195451 68.453) (end 46.195451 68.453) (width 1) (layer B.Cu) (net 7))
 (segment (start 62.103 81.788) (end 60.833 80.518) (width 1) (layer B.Cu) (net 7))
 (segment (start 43.053 62.738) (end 44.323 62.738) (width 1) (layer B.Cu) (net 7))
 (segment (start 62.103 83.058) (end 62.103 81.788) (width 1) (layer B.Cu) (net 7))
 (segment (start 42.481001 67.246001) (end 42.481001 63.309999) (width 1) (layer B.Cu) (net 7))
 (segment (start 52.578 80.518) (end 47.498 75.438) (width 1) (layer B.Cu) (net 7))
 (segment (start 43.688 68.453) (end 42.481001 67.246001) (width 1) (layer B.Cu) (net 7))
 (segment (start 60.833 80.518) (end 52.578 80.518) (width 1) (layer B.Cu) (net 7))
 (segment (start 58.293 80.518) (end 76.708 62.103) (width 1) (layer F.Cu) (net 7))
 (segment (start 76.708 62.103) (end 76.708 62.103) (width 1) (layer F.Cu) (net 7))
 (via (at 76.708 62.103) (size 1.4) (drill 0.8) (layers F.Cu B.Cu) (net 7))
 (segment (start 79.883 65.278) (end 76.708 62.103) (width 1) (layer B.Cu) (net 7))
 (segment (start 82.423 65.278) (end 79.883 65.278) (width 1) (layer B.Cu) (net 7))
 (segment (start 76.708 62.103) (end 74.803 60.198) (width 1) (layer B.Cu) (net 7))
 (segment (start 74.803 60.198) (end 70.993 60.198) (width 1) (layer B.Cu) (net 7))
 (segment (start 46.195451 68.453) (end 43.688 68.453) (width 1) (layer B.Cu) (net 7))
 (via (at 46.195451 68.453) (size 1.4) (drill 0.8) (layers F.Cu B.Cu) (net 7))
 (segment (start 67.818 46.863) (end 69.088 48.133) (width 1) (layer B.Cu) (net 7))
 (segment (start 69.088 48.133) (end 81.153 60.198) (width 1) (layer B.Cu) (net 7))
 (via (at 69.088 48.133) (size 1.4) (drill 0.8) (layers F.Cu B.Cu) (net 7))
 (segment (start 46.863 74.803) (end 52.578 80.518) (width 1) (layer B.Cu) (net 7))
 (segment (start 46.863 69.120549) (end 46.863 74.803) (width 1) (layer B.Cu) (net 7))
 (segment (start 46.863 69.120549) (end 46.195451 68.453) (width 1) (layer B.Cu) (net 7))
 (segment (start 49.094847 60.506153) (end 48.133 59.544306) (width 1) (layer F.Cu) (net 7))
 (segment (start 48.133 59.544306) (end 48.133 58.293) (width 1) (layer F.Cu) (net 7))
 (segment (start 48.133 58.293) (end 59.563 46.863) (width 1) (layer F.Cu) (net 7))
 (segment (start 59.563 46.863) (end 59.563 44.323) (width 1) (layer F.Cu) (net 7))
 (segment (start 60.578001 43.307999) (end 64.262999 43.307999) (width 1) (layer F.Cu) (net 7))
 (segment (start 59.563 44.323) (end 60.578001 43.307999) (width 1) (layer F.Cu) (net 7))
 (segment (start 64.643 43.688) (end 64.643 44.958) (width 1) (layer F.Cu) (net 7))
 (segment (start 64.262999 43.307999) (end 64.643 43.688) (width 1) (layer F.Cu) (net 7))
 (segment (start 49.403 65.278) (end 50.673 64.008) (width 0.5) (layer B.Cu) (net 5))
 (segment (start 49.403 67.183) (end 49.403 65.278) (width 0.5) (layer B.Cu) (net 5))
 (segment (start 53.848 58.075102) (end 52.686949 56.914051) (width 0.5) (layer B.Cu) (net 5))
 (segment (start 53.848 58.928) (end 53.848 58.075102) (width 0.5) (layer B.Cu) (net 5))
 (segment (start 52.578 60.198) (end 53.848 58.928) (width 0.5) (layer B.Cu) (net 5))
 (segment (start 50.673 64.008) (end 52.578 62.103) (width 0.5) (layer B.Cu) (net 5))
 (segment (start 52.578 62.103) (end 52.578 60.198) (width 0.5) (layer B.Cu) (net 5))
 (segment (start 51.976958 73.056168) (end 51.976958 69.756958) (width 0.5) (layer B.Cu) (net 5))
 (segment (start 51.340563 73.692563) (end 51.976958 73.056168) (width 0.5) (layer B.Cu) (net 5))
 (segment (start 51.944395 69.724395) (end 50.927 68.707) (width 0.5) (layer B.Cu) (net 5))
 (segment (start 50.927 68.707) (end 49.403 67.183) (width 0.5) (layer B.Cu) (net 5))
 (segment (start 65.008648 52.032784) (end 66.458216 50.583216) (width 0.5) (layer B.Cu) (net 2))
 (segment (start 64.732784 52.032784) (end 65.008648 52.032784) (width 0.5) (layer B.Cu) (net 2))
 (segment (start 64.1671 52.598468) (end 64.732784 52.032784) (width 0.5) (layer B.Cu) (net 2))
 (segment (start 64.028468 52.598468) (end 64.1671 52.598468) (width 0.5) (layer B.Cu) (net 2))
 (segment (start 64.008 52.578) (end 64.028468 52.598468) (width 0.5) (layer B.Cu) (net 2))
 (segment (start 59.127206 52.578) (end 64.008 52.578) (width 0.5) (layer B.Cu) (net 2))
 (segment (start 58.075103 51.525897) (end 59.127206 52.578) (width 0.5) (layer B.Cu) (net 2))
 (segment (start 75.855103 69.305897) (end 74.367206 67.818) (width 0.5) (layer B.Cu) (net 9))
 (segment (start 74.367206 67.818) (end 72.898 67.818) (width 0.5) (layer B.Cu) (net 9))
 (segment (start 57.004308 68.453) (end 56.061154 69.396154) (width 0.5) (layer B.Cu) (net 9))
 (segment (start 58.293 68.453) (end 57.004308 68.453) (width 0.5) (layer B.Cu) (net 9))
 (segment (start 72.898 67.818) (end 71.12 67.818) (width 0.5) (layer B.Cu) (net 9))
 (segment (start 65.024 73.914) (end 63.754 73.914) (width 0.5) (layer B.Cu) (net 9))
 (segment (start 71.12 67.818) (end 65.024 73.914) (width 0.5) (layer B.Cu) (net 9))
 (segment (start 63.754 73.914) (end 58.293 68.453) (width 0.5) (layer B.Cu) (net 9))
 (segment (start 61.468 74.803) (end 63.373 76.708) (width 0.5) (layer B.Cu) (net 10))
 (segment (start 57.857205 71.192205) (end 61.468 74.803) (width 0.5) (layer B.Cu) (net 10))
 (segment (start 63.373 76.708) (end 64.643 76.708) (width 0.5) (layer B.Cu) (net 10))
 (segment (start 64.643 76.708) (end 65.278 76.708) (width 0.5) (layer B.Cu) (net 10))
 (segment (start 71.734051 70.251949) (end 70.358 71.628) (width 0.5) (layer B.Cu) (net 10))
 (segment (start 73.209053 70.251949) (end 71.734051 70.251949) (width 0.5) (layer B.Cu) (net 10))
 (segment (start 74.059052 71.101948) (end 73.209053 70.251949) (width 0.5) (layer B.Cu) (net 10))
 (segment (start 65.278 76.708) (end 70.358 71.628) (width 0.5) (layer B.Cu) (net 10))
 (segment (start 70.358 71.628) (end 71.628 70.358) (width 0.5) (layer B.Cu) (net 10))
 (segment (start 77.959308 67.818) (end 77.651154 67.509846) (width 0.5) (layer B.Cu) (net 12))
 (segment (start 82.423 67.818) (end 77.959308 67.818) (width 0.5) (layer B.Cu) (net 12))
 (segment (start 59.563 84.408) (end 60.118 84.963) (width 0.5) (layer B.Cu) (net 11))
 (segment (start 59.563 83.058) (end 59.563 84.408) (width 0.5) (layer B.Cu) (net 11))
 (segment (start 60.118 84.963) (end 66.548 84.963) (width 0.5) (layer B.Cu) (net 11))
 (segment (start 66.874847 84.636153) (end 66.874847 78.286153) (width 0.5) (layer B.Cu) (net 11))
 (segment (start 66.548 84.963) (end 66.874847 84.636153) (width 0.5) (layer B.Cu) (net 11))
 (segment (start 44.323 60.198) (end 45.673 60.198) (width 0.5) (layer B.Cu) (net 4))
 (segment (start 51.602999 54.268001) (end 50.118 55.753) (width 0.5) (layer B.Cu) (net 4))
 (segment (start 53.633001 54.268001) (end 51.602999 54.268001) (width 0.5) (layer B.Cu) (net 4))
 (segment (start 54.483 55.118) (end 53.633001 54.268001) (width 0.5) (layer B.Cu) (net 4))
 (segment (start 45.673 60.198) (end 50.118 55.753) (width 0.5) (layer B.Cu) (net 4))
 (segment (start 50.118 55.753) (end 51.388 54.483) (width 0.5) (layer B.Cu) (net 4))
 (segment (start 67.183 43.608) (end 67.183 44.958) (width 0.5) (layer B.Cu) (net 1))
 (segment (start 59.871154 49.729846) (end 59.871154 48.427764) (width 0.5) (layer B.Cu) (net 1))
 (segment (start 59.871154 48.427764) (end 58.928 47.48461) (width 0.5) (layer B.Cu) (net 1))
 (segment (start 58.928 47.48461) (end 58.928 44.323) (width 0.5) (layer B.Cu) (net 1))
 (segment (start 58.928 44.323) (end 60.384999 42.866001) (width 0.5) (layer B.Cu) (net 1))
 (segment (start 60.384999 42.866001) (end 66.441001 42.866001) (width 0.5) (layer B.Cu) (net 1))
 (segment (start 66.441001 42.866001) (end 67.183 43.608) (width 0.5) (layer B.Cu) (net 1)))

